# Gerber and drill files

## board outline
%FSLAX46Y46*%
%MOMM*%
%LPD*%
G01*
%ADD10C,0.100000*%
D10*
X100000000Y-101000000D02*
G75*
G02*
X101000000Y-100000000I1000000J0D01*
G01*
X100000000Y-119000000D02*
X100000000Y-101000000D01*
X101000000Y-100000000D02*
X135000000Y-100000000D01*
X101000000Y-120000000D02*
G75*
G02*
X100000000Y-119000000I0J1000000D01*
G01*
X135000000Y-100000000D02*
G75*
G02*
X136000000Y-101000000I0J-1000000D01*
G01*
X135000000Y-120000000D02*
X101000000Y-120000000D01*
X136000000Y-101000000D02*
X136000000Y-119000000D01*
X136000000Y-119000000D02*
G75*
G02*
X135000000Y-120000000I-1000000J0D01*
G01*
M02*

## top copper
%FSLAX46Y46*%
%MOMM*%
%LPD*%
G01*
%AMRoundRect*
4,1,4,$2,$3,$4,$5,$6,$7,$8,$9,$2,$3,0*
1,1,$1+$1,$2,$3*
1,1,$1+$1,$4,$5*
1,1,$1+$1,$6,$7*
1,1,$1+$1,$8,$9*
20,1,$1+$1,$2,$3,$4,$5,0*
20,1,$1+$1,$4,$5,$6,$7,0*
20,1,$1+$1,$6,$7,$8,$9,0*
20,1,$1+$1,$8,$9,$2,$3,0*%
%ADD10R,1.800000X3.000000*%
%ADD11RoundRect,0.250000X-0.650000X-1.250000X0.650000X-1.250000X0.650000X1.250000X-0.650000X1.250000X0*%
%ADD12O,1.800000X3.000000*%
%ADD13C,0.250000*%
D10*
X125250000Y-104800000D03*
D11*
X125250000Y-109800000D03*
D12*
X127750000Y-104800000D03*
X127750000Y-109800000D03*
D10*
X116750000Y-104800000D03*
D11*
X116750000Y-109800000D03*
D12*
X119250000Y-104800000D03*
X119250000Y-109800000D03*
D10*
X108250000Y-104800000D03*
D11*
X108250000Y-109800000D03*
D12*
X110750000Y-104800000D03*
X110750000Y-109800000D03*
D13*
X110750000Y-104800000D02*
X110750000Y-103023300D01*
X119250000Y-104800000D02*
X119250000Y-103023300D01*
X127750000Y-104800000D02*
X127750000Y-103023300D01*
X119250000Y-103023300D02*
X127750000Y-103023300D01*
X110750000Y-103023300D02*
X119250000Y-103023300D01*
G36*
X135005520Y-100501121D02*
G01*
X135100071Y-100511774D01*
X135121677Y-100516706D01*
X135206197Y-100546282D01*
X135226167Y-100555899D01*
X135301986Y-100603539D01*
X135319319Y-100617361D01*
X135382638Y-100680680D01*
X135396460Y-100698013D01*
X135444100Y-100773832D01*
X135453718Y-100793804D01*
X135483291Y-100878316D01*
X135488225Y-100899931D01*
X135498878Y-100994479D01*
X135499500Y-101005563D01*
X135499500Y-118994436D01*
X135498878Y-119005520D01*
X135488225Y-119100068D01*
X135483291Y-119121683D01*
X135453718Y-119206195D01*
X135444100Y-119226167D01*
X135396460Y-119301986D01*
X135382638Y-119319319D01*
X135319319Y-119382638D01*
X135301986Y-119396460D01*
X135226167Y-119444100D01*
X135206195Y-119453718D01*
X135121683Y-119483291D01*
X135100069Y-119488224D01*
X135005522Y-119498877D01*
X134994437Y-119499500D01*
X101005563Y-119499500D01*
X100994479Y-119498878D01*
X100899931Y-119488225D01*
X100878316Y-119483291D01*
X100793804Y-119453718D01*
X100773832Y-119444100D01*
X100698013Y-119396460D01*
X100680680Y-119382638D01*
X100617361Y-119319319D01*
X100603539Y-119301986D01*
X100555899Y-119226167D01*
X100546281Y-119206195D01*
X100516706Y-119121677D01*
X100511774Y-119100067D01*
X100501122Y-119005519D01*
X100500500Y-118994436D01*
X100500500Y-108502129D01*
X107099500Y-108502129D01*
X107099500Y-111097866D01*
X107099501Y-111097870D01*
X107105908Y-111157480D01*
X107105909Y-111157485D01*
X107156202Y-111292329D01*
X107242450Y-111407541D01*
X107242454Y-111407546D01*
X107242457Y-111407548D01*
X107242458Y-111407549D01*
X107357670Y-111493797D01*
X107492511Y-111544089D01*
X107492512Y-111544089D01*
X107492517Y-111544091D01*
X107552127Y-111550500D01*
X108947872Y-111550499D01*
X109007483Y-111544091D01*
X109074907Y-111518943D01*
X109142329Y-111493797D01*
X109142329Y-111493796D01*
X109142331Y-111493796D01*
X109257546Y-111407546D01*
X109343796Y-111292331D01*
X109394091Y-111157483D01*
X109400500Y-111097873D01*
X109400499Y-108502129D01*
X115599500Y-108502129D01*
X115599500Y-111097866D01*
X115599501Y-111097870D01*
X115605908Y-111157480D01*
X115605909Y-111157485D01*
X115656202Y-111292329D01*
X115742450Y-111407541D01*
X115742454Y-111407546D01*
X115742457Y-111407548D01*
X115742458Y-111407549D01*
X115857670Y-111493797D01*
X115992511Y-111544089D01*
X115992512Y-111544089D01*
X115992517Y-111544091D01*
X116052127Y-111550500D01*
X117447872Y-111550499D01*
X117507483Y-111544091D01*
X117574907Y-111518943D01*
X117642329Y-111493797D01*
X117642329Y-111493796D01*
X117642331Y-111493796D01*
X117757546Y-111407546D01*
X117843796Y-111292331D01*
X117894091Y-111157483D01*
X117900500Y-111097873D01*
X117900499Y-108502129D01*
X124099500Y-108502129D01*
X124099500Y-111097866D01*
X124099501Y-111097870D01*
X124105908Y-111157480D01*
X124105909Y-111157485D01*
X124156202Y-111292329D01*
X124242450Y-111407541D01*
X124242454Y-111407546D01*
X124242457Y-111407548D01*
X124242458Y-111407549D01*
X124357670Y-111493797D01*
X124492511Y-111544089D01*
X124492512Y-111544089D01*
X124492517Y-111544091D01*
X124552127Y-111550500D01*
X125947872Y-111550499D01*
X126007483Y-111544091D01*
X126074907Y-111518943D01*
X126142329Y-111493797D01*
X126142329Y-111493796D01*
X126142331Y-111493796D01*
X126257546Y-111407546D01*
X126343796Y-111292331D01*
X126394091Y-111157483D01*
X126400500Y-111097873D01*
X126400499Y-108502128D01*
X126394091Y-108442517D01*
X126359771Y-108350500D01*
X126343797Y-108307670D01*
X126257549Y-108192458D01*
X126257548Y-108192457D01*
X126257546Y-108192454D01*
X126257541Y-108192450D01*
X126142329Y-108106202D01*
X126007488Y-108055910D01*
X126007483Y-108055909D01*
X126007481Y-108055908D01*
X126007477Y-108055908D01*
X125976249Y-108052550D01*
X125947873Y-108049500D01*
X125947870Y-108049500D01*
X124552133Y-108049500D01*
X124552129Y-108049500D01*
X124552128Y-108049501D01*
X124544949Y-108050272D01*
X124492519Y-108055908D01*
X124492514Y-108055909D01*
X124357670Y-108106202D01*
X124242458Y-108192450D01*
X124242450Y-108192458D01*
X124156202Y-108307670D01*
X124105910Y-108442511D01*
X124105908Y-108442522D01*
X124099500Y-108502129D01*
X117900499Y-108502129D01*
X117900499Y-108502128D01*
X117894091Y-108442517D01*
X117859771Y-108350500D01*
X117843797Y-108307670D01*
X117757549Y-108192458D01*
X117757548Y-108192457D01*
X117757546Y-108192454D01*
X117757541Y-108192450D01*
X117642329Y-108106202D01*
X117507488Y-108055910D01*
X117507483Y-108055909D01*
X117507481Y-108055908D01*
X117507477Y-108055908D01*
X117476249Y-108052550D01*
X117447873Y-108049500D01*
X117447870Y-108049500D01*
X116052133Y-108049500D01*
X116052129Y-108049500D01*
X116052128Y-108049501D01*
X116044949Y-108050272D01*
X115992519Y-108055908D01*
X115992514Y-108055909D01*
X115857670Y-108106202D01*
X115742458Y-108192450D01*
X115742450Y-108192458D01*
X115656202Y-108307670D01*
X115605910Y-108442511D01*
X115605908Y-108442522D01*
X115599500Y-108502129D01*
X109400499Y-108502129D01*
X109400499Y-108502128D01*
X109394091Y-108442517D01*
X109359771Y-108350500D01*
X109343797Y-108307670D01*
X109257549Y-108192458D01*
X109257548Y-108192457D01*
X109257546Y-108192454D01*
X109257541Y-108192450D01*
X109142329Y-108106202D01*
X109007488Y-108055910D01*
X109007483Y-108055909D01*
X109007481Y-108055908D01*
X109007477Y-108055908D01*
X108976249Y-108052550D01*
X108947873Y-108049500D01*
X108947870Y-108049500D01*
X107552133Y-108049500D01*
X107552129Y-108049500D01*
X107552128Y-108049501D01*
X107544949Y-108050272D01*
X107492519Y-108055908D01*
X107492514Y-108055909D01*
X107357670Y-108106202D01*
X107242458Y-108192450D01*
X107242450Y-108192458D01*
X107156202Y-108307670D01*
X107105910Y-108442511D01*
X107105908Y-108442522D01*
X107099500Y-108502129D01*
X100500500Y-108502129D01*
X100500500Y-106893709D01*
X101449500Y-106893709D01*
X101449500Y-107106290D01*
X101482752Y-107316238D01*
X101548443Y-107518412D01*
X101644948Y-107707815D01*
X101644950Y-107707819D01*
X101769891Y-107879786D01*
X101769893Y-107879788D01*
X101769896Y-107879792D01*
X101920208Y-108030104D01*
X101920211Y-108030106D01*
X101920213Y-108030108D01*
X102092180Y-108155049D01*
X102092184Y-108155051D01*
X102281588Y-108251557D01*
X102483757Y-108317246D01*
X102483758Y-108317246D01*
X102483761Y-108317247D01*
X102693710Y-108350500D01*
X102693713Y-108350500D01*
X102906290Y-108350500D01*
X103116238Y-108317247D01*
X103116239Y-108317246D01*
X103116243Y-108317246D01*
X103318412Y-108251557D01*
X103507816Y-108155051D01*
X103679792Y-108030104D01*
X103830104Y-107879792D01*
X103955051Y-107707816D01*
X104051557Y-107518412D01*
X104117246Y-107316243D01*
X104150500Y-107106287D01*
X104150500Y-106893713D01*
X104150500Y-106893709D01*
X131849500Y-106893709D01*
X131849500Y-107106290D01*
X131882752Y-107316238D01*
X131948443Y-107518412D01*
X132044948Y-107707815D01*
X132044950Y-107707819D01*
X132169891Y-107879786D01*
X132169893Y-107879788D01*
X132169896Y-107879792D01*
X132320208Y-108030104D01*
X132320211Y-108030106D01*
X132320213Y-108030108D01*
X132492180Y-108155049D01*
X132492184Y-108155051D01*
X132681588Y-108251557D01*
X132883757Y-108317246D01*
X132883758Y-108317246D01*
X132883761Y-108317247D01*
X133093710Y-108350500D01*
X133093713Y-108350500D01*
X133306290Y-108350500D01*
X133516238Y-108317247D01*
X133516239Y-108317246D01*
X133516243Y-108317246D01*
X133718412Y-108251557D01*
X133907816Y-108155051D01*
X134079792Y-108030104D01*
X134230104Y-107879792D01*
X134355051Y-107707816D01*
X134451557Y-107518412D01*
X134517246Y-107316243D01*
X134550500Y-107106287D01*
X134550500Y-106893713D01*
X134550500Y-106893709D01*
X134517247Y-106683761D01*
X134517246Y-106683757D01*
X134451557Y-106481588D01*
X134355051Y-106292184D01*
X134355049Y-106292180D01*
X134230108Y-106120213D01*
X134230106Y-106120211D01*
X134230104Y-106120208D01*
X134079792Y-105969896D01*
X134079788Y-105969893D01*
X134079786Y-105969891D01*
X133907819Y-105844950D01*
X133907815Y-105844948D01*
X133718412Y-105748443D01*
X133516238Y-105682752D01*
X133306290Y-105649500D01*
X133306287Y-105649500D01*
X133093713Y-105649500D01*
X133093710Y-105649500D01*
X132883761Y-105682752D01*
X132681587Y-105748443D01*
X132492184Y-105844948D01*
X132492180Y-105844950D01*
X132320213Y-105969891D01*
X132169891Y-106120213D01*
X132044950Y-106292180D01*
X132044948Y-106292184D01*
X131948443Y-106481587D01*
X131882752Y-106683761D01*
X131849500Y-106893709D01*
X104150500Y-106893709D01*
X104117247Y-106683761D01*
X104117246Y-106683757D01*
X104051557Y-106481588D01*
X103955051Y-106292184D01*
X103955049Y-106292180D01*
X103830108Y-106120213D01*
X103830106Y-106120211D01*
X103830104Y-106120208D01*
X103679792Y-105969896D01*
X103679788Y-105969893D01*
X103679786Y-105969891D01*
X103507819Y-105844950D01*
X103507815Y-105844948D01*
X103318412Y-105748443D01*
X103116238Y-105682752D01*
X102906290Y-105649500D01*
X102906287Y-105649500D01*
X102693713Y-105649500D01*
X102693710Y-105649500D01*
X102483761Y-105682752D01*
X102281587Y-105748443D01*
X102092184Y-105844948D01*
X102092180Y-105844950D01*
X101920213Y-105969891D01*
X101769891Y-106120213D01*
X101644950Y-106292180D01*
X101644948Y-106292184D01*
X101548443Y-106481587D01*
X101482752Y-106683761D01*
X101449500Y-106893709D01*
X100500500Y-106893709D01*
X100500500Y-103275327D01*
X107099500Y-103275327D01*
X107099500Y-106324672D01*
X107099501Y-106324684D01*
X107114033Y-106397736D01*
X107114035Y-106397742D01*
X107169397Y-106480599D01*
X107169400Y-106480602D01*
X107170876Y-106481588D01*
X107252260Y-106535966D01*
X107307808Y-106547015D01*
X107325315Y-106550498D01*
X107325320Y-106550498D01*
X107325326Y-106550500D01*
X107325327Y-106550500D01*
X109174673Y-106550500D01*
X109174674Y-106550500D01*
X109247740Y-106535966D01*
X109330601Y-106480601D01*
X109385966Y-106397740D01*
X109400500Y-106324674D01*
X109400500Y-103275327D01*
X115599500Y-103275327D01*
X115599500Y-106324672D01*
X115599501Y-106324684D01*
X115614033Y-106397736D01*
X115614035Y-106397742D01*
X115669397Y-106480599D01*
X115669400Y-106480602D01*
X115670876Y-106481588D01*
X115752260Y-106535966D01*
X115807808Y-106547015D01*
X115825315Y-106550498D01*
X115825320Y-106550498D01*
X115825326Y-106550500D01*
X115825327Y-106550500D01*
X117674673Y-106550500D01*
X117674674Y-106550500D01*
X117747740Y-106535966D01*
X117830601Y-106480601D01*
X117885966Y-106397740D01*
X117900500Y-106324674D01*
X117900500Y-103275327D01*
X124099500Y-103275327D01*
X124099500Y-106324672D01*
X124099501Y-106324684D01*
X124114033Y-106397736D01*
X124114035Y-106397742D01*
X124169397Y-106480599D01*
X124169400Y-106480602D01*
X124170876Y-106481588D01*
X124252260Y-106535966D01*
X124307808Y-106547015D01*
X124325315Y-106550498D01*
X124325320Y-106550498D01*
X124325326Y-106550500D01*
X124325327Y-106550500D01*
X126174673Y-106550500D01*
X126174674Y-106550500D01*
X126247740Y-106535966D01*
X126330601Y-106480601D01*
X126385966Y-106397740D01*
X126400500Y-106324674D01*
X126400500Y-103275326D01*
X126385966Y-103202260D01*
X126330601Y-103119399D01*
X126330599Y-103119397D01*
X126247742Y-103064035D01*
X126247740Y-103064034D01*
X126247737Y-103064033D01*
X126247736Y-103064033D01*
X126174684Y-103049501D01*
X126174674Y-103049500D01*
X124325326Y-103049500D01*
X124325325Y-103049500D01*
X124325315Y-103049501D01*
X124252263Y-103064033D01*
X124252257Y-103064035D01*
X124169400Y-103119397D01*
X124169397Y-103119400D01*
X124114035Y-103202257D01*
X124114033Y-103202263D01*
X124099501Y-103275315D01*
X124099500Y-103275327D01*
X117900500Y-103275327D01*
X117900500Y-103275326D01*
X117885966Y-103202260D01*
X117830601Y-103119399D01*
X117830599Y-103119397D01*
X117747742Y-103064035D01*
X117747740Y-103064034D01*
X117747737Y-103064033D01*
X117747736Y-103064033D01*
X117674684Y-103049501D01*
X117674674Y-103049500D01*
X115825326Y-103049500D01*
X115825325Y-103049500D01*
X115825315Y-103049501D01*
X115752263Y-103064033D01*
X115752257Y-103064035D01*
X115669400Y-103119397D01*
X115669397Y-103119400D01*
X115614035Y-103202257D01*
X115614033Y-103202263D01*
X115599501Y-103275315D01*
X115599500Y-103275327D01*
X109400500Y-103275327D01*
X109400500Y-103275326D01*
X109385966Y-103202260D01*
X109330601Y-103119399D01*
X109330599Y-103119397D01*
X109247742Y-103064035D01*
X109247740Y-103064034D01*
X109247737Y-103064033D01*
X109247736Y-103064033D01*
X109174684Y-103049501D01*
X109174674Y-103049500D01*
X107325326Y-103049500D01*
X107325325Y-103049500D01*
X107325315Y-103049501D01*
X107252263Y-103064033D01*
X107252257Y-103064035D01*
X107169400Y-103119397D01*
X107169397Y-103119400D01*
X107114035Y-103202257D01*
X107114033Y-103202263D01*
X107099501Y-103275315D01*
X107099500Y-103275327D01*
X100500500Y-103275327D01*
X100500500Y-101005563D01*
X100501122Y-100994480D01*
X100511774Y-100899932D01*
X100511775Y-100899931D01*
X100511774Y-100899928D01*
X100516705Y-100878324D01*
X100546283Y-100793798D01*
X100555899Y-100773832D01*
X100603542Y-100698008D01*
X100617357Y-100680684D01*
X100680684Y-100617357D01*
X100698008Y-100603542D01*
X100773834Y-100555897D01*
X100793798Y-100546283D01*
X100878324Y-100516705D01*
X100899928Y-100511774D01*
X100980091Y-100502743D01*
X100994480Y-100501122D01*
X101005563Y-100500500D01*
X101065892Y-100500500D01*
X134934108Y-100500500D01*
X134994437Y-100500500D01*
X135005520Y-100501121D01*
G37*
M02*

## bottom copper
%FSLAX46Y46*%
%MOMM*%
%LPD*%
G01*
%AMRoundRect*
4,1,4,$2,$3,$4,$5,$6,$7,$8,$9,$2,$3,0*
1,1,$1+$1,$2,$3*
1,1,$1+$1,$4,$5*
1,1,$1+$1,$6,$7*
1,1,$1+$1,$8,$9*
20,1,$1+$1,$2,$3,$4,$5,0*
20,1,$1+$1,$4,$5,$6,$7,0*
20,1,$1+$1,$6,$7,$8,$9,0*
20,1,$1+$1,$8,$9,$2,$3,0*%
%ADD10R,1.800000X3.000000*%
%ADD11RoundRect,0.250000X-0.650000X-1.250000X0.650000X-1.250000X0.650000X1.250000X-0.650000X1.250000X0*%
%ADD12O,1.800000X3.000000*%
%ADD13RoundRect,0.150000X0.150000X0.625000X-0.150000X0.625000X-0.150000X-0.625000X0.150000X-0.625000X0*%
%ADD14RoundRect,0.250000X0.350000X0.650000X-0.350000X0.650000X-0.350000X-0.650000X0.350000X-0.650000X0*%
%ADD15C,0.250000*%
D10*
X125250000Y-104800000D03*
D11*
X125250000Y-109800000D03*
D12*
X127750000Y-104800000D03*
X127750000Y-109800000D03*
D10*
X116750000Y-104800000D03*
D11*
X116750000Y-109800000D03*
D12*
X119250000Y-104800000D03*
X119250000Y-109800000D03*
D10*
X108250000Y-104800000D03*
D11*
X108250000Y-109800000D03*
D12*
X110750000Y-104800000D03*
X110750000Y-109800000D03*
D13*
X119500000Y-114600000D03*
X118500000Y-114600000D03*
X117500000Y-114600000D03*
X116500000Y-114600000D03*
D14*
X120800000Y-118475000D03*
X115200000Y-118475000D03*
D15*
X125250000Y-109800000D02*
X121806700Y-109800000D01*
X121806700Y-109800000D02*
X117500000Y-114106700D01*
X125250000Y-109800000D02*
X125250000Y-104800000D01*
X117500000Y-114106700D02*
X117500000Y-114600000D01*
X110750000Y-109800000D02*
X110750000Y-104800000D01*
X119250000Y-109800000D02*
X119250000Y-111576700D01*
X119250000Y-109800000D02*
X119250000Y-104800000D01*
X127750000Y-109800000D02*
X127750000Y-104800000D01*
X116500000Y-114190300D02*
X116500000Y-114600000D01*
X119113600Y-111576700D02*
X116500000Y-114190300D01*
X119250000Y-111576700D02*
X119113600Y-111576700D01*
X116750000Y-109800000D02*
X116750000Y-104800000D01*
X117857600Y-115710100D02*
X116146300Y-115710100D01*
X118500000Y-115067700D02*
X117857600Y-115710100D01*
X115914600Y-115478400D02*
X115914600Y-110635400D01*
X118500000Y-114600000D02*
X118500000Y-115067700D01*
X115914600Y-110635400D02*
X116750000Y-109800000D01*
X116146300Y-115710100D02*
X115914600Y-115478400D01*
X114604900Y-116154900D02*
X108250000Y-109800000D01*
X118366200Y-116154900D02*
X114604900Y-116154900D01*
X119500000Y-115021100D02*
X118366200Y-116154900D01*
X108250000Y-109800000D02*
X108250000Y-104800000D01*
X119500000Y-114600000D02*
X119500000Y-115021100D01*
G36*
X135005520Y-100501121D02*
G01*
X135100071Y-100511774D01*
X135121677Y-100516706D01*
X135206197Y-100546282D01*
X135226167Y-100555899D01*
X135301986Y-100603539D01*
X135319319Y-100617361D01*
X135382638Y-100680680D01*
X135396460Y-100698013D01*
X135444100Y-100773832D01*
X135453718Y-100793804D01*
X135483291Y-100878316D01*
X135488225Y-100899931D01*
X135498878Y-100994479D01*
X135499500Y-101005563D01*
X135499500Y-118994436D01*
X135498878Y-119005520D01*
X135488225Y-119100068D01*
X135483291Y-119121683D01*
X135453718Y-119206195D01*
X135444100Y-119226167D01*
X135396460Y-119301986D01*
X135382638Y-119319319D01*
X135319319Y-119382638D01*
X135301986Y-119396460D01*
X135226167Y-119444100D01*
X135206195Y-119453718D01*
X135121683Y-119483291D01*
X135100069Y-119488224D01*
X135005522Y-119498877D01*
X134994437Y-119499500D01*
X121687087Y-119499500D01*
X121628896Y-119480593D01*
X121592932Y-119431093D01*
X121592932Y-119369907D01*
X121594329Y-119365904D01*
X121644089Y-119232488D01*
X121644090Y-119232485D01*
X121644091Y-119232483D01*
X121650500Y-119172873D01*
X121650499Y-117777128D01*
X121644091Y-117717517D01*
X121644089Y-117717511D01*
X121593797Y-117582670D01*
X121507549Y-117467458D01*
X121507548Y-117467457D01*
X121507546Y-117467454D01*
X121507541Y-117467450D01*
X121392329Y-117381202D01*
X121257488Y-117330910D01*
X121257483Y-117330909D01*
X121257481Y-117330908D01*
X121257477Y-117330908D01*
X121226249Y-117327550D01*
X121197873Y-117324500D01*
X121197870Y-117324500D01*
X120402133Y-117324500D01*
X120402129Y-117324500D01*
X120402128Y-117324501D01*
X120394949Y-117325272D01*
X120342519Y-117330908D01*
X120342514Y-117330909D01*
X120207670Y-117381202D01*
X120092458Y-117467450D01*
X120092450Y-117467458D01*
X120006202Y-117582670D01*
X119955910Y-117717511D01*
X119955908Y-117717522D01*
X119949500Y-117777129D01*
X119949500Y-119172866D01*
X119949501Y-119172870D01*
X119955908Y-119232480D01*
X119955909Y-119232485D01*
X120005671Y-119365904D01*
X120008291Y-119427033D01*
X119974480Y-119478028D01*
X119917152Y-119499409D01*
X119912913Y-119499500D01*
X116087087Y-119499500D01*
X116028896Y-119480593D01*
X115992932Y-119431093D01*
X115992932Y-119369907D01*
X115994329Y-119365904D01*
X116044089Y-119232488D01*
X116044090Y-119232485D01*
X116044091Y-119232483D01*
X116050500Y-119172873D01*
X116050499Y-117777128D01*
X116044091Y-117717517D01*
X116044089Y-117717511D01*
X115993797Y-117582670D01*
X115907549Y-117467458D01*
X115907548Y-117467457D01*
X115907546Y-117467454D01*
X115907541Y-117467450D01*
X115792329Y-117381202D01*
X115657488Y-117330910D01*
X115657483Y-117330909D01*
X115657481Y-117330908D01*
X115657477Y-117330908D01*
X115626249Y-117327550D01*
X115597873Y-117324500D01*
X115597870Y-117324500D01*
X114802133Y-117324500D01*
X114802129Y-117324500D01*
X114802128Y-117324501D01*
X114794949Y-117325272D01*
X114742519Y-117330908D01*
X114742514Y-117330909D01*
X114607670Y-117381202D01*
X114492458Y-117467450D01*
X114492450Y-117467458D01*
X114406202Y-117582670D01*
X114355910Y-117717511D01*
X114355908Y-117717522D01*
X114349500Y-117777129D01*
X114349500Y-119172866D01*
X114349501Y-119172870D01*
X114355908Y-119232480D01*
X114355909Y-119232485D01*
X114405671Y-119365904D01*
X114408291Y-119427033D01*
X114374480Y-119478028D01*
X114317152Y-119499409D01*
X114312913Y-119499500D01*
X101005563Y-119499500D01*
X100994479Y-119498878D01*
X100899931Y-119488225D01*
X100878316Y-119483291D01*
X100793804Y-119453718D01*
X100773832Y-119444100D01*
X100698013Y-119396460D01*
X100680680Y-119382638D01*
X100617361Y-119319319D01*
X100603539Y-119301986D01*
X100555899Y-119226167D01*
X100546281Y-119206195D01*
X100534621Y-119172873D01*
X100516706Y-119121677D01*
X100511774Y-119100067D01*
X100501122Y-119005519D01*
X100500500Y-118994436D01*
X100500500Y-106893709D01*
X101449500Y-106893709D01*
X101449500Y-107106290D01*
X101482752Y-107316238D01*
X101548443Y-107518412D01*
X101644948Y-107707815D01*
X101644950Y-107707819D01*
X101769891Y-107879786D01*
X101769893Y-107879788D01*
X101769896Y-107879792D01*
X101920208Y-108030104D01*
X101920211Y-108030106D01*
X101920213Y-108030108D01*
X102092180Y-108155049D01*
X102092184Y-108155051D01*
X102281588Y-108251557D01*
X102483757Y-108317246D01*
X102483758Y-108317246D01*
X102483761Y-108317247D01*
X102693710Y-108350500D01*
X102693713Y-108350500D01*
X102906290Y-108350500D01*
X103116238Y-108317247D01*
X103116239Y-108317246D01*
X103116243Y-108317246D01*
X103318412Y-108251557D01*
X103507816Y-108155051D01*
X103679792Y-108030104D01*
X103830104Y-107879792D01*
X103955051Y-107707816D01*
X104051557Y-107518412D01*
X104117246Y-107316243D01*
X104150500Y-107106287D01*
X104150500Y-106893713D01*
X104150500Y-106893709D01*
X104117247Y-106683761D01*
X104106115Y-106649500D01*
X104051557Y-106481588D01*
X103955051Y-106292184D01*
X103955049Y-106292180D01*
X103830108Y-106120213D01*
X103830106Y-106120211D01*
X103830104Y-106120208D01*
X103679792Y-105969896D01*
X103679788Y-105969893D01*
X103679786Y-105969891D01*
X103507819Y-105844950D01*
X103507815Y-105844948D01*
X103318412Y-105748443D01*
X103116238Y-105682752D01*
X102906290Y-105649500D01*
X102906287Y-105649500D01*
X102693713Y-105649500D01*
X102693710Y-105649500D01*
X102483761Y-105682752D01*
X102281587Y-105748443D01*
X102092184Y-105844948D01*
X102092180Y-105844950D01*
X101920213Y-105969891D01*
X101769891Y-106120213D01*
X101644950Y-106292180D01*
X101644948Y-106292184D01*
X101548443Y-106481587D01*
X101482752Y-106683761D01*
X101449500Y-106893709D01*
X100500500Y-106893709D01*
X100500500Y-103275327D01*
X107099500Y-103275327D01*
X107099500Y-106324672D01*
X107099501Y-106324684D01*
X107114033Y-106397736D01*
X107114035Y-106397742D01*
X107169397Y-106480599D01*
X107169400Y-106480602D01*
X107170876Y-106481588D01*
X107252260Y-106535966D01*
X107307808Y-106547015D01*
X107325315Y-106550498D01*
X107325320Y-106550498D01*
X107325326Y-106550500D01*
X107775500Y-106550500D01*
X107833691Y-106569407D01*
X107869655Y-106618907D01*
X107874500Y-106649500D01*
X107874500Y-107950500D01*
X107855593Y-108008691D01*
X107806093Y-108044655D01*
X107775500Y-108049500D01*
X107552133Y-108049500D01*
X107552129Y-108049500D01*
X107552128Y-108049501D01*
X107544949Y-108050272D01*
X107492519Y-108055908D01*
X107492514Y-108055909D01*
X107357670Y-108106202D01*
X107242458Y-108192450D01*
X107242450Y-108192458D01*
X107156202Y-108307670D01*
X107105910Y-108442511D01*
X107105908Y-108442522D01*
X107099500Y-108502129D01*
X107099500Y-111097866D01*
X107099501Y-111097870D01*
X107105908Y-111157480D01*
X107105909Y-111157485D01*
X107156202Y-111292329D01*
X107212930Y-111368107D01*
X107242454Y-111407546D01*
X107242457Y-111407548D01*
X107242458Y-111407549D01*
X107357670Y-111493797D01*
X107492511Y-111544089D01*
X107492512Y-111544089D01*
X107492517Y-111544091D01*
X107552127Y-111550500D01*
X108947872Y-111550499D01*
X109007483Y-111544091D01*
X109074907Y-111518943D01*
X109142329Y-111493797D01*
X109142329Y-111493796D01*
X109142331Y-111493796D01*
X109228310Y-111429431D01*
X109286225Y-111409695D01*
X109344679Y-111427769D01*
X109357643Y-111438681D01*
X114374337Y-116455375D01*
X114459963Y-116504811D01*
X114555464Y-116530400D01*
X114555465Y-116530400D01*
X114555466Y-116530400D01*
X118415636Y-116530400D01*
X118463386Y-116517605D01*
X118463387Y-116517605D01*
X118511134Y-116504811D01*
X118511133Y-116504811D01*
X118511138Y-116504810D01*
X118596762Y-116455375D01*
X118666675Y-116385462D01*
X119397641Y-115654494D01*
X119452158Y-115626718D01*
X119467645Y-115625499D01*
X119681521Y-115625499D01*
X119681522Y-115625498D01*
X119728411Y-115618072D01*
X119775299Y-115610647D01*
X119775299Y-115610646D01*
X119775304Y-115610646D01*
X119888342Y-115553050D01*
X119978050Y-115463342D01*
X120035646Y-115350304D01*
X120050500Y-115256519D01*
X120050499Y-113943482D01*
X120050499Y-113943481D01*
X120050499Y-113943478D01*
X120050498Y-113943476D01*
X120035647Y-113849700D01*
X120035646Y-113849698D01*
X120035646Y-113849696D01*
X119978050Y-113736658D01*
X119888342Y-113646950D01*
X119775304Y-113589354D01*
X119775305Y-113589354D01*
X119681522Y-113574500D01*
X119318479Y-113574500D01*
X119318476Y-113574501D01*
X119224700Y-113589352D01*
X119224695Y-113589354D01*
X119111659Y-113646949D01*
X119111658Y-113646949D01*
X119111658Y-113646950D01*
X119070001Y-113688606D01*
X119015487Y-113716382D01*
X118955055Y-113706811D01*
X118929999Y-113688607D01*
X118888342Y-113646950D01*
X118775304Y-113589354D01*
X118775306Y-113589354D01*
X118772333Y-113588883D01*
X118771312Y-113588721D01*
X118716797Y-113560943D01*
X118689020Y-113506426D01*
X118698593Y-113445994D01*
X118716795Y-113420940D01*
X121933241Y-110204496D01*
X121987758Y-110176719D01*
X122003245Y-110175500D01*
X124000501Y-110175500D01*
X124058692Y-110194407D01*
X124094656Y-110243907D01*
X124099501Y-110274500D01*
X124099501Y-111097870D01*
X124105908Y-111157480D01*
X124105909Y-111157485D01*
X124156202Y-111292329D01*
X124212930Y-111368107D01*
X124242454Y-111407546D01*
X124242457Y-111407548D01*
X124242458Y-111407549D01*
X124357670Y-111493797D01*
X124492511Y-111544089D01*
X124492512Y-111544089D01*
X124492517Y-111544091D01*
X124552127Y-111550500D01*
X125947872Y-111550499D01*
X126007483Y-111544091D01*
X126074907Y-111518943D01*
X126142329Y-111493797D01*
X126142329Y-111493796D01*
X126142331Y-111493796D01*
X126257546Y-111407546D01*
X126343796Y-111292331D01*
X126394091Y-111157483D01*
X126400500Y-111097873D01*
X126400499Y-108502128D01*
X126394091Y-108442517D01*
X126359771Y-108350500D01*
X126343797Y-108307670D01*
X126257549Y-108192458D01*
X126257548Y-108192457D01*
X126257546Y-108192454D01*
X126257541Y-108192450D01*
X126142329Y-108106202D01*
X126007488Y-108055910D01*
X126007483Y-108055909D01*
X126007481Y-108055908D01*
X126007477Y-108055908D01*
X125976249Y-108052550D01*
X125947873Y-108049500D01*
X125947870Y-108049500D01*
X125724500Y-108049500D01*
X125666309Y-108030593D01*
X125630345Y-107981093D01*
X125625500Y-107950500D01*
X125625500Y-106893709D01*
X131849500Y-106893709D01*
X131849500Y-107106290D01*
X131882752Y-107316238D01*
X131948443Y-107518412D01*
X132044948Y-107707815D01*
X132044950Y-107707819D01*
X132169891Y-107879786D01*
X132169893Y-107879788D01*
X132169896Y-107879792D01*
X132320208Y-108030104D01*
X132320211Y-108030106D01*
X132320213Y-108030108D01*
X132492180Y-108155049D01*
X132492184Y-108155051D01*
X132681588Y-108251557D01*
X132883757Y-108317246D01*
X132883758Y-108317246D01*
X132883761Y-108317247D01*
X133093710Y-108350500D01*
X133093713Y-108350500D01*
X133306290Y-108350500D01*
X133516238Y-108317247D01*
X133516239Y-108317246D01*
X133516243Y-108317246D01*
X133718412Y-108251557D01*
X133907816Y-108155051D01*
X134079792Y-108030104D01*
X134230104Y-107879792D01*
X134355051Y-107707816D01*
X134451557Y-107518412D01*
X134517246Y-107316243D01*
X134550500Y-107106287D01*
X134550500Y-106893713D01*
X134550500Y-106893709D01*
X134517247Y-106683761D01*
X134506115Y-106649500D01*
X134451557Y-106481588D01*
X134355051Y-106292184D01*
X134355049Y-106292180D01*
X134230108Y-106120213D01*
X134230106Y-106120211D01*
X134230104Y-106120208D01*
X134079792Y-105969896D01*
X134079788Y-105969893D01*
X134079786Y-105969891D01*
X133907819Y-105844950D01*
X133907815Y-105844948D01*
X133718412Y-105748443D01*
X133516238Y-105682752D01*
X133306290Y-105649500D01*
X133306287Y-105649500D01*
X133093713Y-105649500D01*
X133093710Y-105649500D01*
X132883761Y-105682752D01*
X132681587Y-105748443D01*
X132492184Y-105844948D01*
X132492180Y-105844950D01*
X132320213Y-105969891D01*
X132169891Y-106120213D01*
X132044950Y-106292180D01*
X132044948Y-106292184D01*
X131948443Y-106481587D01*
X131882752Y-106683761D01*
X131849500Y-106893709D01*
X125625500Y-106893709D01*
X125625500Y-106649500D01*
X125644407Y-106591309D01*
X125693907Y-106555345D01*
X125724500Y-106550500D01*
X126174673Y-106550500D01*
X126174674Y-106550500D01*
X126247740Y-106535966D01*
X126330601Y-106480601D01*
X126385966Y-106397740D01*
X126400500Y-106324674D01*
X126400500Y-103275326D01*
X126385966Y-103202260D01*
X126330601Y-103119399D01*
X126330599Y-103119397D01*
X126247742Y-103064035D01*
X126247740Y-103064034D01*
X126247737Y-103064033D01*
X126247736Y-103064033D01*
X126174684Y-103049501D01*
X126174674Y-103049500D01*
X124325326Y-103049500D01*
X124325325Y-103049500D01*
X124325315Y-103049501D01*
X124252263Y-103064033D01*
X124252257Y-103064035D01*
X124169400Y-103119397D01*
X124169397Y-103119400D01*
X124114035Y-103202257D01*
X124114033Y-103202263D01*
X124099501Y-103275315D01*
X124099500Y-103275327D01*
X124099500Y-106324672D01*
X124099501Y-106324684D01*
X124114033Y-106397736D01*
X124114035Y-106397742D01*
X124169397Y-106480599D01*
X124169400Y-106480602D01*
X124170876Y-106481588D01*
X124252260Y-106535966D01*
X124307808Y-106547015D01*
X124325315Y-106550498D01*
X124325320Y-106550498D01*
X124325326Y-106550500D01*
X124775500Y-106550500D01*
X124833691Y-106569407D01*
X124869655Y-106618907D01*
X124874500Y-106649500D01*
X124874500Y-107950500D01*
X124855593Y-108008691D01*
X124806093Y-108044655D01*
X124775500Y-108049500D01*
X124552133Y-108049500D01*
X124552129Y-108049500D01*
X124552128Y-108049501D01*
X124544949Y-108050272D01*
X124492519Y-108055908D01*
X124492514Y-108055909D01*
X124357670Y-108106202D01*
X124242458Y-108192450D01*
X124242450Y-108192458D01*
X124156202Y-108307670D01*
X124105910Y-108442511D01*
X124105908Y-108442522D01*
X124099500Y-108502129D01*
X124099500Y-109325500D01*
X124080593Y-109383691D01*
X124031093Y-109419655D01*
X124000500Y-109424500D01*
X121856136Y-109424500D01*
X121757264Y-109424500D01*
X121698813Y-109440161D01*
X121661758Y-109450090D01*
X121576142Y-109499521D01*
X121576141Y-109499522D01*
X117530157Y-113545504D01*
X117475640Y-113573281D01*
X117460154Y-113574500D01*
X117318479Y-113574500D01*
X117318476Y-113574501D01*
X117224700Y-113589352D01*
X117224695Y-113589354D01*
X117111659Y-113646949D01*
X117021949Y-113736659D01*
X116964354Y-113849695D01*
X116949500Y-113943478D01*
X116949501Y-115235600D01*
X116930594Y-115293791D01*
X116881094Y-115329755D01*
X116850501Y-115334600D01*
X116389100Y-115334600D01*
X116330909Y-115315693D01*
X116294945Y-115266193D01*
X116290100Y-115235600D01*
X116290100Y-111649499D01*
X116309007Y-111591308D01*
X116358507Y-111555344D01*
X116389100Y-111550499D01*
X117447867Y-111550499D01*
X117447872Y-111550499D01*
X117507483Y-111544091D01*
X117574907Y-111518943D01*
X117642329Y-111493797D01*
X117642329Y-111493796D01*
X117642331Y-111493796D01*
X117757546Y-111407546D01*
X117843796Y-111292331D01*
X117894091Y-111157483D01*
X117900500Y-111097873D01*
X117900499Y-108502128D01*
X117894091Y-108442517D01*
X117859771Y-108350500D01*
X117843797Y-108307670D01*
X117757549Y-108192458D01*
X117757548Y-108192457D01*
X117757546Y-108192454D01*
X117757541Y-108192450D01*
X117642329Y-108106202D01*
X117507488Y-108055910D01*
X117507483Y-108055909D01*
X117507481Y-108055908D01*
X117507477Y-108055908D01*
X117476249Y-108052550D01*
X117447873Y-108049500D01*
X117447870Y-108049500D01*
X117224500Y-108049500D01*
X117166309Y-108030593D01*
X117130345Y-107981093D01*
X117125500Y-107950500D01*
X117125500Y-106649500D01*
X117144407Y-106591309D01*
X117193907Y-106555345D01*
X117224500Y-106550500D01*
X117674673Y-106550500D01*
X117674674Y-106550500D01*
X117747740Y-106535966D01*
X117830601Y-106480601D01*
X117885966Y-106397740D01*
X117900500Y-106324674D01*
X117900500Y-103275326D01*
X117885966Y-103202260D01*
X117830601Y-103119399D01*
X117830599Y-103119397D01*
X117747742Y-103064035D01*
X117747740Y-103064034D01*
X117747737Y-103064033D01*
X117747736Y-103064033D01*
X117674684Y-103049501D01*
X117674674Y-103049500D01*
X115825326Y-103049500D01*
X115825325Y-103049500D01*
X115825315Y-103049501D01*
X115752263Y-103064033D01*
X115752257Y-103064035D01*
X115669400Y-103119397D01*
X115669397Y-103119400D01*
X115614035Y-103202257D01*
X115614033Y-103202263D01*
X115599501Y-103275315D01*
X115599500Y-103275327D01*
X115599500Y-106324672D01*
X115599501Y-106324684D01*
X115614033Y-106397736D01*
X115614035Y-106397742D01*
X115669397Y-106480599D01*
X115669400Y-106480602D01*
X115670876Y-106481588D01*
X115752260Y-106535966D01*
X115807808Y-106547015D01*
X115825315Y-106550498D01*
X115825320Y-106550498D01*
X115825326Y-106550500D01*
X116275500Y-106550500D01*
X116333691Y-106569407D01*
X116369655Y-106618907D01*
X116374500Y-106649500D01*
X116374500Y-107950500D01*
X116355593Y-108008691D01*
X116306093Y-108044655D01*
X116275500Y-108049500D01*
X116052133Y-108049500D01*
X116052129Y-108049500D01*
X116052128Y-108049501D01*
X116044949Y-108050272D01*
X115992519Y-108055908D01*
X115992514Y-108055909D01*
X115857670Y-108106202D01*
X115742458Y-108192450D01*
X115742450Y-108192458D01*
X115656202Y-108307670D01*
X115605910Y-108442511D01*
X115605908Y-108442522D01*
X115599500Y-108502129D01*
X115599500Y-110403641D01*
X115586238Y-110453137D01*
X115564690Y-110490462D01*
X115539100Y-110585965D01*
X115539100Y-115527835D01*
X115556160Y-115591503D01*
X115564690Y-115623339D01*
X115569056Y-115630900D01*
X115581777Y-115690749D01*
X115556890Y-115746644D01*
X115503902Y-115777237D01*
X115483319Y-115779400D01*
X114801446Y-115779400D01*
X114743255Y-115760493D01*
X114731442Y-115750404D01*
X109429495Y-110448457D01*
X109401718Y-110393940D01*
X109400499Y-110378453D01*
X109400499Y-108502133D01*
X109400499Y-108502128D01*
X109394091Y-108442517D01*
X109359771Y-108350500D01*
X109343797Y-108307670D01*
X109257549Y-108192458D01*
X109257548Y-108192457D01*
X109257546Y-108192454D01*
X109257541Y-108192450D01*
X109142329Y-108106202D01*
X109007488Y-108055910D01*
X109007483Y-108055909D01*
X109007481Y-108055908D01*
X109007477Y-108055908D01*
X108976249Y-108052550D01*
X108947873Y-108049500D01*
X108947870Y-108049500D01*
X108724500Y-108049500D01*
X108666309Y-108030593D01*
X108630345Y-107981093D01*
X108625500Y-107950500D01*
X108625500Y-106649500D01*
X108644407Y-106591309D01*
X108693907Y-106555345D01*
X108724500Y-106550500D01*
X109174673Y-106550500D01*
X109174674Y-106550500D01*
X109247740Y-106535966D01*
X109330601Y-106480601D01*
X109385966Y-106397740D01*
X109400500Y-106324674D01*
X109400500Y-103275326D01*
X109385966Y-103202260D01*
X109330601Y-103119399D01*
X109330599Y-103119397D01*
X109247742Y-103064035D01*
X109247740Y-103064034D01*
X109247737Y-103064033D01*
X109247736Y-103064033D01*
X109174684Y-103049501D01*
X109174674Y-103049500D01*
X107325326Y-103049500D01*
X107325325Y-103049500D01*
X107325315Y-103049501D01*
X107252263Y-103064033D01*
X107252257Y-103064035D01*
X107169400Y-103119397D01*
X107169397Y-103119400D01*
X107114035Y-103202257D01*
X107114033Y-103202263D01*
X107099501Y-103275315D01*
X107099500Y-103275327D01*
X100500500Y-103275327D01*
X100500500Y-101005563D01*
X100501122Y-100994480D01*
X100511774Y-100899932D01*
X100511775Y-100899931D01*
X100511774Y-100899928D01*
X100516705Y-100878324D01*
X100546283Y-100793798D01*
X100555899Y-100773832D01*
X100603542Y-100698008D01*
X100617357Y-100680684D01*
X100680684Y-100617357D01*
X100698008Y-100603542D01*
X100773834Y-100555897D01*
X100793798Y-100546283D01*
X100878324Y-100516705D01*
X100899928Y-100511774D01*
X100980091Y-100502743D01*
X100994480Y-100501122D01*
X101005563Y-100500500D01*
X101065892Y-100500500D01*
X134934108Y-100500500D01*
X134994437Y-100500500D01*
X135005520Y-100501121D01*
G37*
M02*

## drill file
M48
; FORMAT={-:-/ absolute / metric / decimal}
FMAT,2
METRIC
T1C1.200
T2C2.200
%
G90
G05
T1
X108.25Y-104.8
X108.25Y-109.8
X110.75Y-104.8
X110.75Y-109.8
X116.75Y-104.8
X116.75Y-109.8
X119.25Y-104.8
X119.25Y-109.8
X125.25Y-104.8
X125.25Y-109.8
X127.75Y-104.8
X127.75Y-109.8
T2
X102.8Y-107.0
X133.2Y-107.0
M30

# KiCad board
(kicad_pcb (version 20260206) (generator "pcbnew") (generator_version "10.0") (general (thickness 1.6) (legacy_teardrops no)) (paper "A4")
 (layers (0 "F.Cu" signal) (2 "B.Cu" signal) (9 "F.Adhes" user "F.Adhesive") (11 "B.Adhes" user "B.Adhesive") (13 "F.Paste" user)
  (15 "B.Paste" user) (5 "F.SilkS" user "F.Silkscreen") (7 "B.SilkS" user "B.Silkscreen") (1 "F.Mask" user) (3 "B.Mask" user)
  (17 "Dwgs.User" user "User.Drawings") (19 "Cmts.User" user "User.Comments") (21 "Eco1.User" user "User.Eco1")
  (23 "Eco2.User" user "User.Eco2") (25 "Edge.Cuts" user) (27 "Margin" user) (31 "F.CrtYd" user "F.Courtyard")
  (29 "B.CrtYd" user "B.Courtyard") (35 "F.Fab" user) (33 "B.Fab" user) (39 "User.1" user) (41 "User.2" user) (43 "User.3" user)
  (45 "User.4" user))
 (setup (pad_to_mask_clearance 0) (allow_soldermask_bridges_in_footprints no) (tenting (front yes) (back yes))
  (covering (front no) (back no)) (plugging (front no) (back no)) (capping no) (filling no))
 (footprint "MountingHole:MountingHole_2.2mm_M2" (layer "F.Cu") (at 102.8 107)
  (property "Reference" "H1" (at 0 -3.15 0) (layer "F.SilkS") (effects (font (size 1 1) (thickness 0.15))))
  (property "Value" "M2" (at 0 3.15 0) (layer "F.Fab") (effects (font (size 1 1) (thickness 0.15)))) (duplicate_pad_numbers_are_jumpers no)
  (pad "" np_thru_hole circle (at 0 0) (size 2.2 2.2) (drill 2.2) (layers "*.Cu" "*.Mask") (zone_connect 2)))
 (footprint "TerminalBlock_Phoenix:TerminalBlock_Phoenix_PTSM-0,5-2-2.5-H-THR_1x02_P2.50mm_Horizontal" (layer "F.Cu") (at 125.25 109.8)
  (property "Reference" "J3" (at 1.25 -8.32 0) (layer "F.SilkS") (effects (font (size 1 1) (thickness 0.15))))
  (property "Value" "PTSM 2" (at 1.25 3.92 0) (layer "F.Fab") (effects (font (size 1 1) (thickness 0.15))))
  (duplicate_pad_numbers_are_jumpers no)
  (pad "1" thru_hole rect (at 0 -5) (size 1.8 3) (drill 1.2) (layers "*.Cu" "*.Mask") (remove_unused_layers no) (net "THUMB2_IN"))
  (pad "1" thru_hole roundrect (at 0 0) (size 1.8 3) (drill 1.2) (layers "*.Cu" "*.Mask") (remove_unused_layers no)
   (roundrect_rratio 0.138889) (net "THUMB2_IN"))
  (pad "2" thru_hole oval (at 2.5 -5) (size 1.8 3) (drill 1.2) (layers "*.Cu" "*.Mask") (remove_unused_layers no) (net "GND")
   (zone_connect 2))
  (pad "2" thru_hole oval (at 2.5 0) (size 1.8 3) (drill 1.2) (layers "*.Cu" "*.Mask") (remove_unused_layers no) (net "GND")
   (zone_connect 2)))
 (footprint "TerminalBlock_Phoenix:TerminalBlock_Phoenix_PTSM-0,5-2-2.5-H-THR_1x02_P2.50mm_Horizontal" (layer "F.Cu") (at 116.75 109.8)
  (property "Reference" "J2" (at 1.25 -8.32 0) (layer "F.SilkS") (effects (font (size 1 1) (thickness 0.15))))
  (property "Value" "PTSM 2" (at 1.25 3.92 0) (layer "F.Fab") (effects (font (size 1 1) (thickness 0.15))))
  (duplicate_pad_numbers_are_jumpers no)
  (pad "1" thru_hole rect (at 0 -5) (size 1.8 3) (drill 1.2) (layers "*.Cu" "*.Mask") (remove_unused_layers no) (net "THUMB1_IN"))
  (pad "1" thru_hole roundrect (at 0 0) (size 1.8 3) (drill 1.2) (layers "*.Cu" "*.Mask") (remove_unused_layers no)
   (roundrect_rratio 0.138889) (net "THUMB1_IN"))
  (pad "2" thru_hole oval (at 2.5 -5) (size 1.8 3) (drill 1.2) (layers "*.Cu" "*.Mask") (remove_unused_layers no) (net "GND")
   (zone_connect 2))
  (pad "2" thru_hole oval (at 2.5 0) (size 1.8 3) (drill 1.2) (layers "*.Cu" "*.Mask") (remove_unused_layers no) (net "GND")
   (zone_connect 2)))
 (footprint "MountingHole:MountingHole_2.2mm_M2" (layer "F.Cu") (at 133.2 107)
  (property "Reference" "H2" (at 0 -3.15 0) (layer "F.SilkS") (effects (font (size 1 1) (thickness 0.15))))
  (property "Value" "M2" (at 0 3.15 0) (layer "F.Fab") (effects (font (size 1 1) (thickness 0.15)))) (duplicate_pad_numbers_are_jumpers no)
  (pad "" np_thru_hole circle (at 0 0) (size 2.2 2.2) (drill 2.2) (layers "*.Cu" "*.Mask") (zone_connect 2)))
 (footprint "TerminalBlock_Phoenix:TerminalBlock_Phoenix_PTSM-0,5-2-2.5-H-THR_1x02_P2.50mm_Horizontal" (layer "F.Cu") (at 108.25 109.8)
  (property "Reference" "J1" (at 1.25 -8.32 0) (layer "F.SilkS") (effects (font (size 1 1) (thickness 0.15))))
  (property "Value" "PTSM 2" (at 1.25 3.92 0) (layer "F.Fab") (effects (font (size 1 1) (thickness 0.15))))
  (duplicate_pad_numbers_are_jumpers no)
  (pad "1" thru_hole rect (at 0 -5) (size 1.8 3) (drill 1.2) (layers "*.Cu" "*.Mask") (remove_unused_layers no) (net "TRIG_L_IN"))
  (pad "1" thru_hole roundrect (at 0 0) (size 1.8 3) (drill 1.2) (layers "*.Cu" "*.Mask") (remove_unused_layers no)
   (roundrect_rratio 0.138889) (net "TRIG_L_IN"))
  (pad "2" thru_hole oval (at 2.5 -5) (size 1.8 3) (drill 1.2) (layers "*.Cu" "*.Mask") (remove_unused_layers no) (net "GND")
   (zone_connect 2))
  (pad "2" thru_hole oval (at 2.5 0) (size 1.8 3) (drill 1.2) (layers "*.Cu" "*.Mask") (remove_unused_layers no) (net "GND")
   (zone_connect 2)))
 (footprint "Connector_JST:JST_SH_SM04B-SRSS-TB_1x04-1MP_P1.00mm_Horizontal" (layer "B.Cu") (at 118 116.6 180)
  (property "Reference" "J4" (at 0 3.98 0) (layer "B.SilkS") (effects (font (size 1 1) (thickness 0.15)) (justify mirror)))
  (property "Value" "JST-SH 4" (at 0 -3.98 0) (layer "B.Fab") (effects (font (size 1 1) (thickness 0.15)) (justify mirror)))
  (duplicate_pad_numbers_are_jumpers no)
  (pad "1" smd roundrect (at -1.5 2 180) (size 0.6 1.55) (layers "B.Cu" "B.Mask" "B.Paste") (roundrect_rratio 0.25) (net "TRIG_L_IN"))
  (pad "2" smd roundrect (at -0.5 2 180) (size 0.6 1.55) (layers "B.Cu" "B.Mask" "B.Paste") (roundrect_rratio 0.25) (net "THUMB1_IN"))
  (pad "3" smd roundrect (at 0.5 2 180) (size 0.6 1.55) (layers "B.Cu" "B.Mask" "B.Paste") (roundrect_rratio 0.25) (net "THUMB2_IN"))
  (pad "4" smd roundrect (at 1.5 2 180) (size 0.6 1.55) (layers "B.Cu" "B.Mask" "B.Paste") (roundrect_rratio 0.25) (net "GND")
   (zone_connect 2))
  (pad "MP" smd roundrect (at -2.8 -1.875 180) (size 1.2 1.8) (layers "B.Cu" "B.Mask" "B.Paste") (roundrect_rratio 0.208333)
   (zone_connect 2))
  (pad "MP" smd roundrect (at 2.8 -1.875 180) (size 1.2 1.8) (layers "B.Cu" "B.Mask" "B.Paste") (roundrect_rratio 0.208333) (zone_connect 2)))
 (gr_arc (start 100 101) (mid 100.292893 100.292893) (end 101 100) (stroke (width 0.1) (type default)) (layer "Edge.Cuts"))
 (gr_line (start 100 119) (end 100 101) (stroke (width 0.1) (type default)) (layer "Edge.Cuts"))
 (gr_line (start 101 100) (end 135 100) (stroke (width 0.1) (type default)) (layer "Edge.Cuts"))
 (gr_arc (start 101 120) (mid 100.292893 119.707107) (end 100 119) (stroke (width 0.1) (type default)) (layer "Edge.Cuts"))
 (gr_arc (start 135 100) (mid 135.707107 100.292893) (end 136 101) (stroke (width 0.1) (type default)) (layer "Edge.Cuts"))
 (gr_line (start 135 120) (end 101 120) (stroke (width 0.1) (type default)) (layer "Edge.Cuts"))
 (gr_line (start 136 101) (end 136 119) (stroke (width 0.1) (type default)) (layer "Edge.Cuts"))
 (gr_arc (start 136 119) (mid 135.707107 119.707107) (end 135 120) (stroke (width 0.1) (type default)) (layer "Edge.Cuts"))
 (segment (start 125.25 109.8) (end 121.8067 109.8) (width 0.25) (layer "B.Cu") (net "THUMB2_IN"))
 (segment (start 121.8067 109.8) (end 117.5 114.1067) (width 0.25) (layer "B.Cu") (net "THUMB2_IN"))
 (segment (start 125.25 109.8) (end 125.25 104.8) (width 0.25) (layer "B.Cu") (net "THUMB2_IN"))
 (segment (start 117.5 114.1067) (end 117.5 114.6) (width 0.25) (layer "B.Cu") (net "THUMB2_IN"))
 (segment (start 110.75 104.8) (end 110.75 103.0233) (width 0.25) (layer "F.Cu") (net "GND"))
 (segment (start 119.25 104.8) (end 119.25 103.0233) (width 0.25) (layer "F.Cu") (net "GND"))
 (segment (start 127.75 104.8) (end 127.75 103.0233) (width 0.25) (layer "F.Cu") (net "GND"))
 (segment (start 119.25 103.0233) (end 127.75 103.0233) (width 0.25) (layer "F.Cu") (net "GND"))
 (segment (start 110.75 103.0233) (end 119.25 103.0233) (width 0.25) (layer "F.Cu") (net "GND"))
 (segment (start 110.75 109.8) (end 110.75 104.8) (width 0.25) (layer "B.Cu") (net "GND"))
 (segment (start 119.25 109.8) (end 119.25 111.5767) (width 0.25) (layer "B.Cu") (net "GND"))
 (segment (start 119.25 109.8) (end 119.25 104.8) (width 0.25) (layer "B.Cu") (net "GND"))
 (segment (start 127.75 109.8) (end 127.75 104.8) (width 0.25) (layer "B.Cu") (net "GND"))
 (segment (start 116.5 114.1903) (end 116.5 114.6) (width 0.25) (layer "B.Cu") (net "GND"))
 (segment (start 119.1136 111.5767) (end 116.5 114.1903) (width 0.25) (layer "B.Cu") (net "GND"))
 (segment (start 119.25 111.5767) (end 119.1136 111.5767) (width 0.25) (layer "B.Cu") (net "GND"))
 (segment (start 116.75 109.8) (end 116.75 104.8) (width 0.25) (layer "B.Cu") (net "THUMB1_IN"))
 (segment (start 117.8576 115.7101) (end 116.1463 115.7101) (width 0.25) (layer "B.Cu") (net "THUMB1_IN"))
 (segment (start 118.5 115.0677) (end 117.8576 115.7101) (width 0.25) (layer "B.Cu") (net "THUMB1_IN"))
 (segment (start 115.9146 115.4784) (end 115.9146 110.6354) (width 0.25) (layer "B.Cu") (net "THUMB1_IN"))
 (segment (start 118.5 114.6) (end 118.5 115.0677) (width 0.25) (layer "B.Cu") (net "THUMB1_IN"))
 (segment (start 115.9146 110.6354) (end 116.75 109.8) (width 0.25) (layer "B.Cu") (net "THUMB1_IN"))
 (segment (start 116.1463 115.7101) (end 115.9146 115.4784) (width 0.25) (layer "B.Cu") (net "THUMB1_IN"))
 (segment (start 114.6049 116.1549) (end 108.25 109.8) (width 0.25) (layer "B.Cu") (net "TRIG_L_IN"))
 (segment (start 118.3662 116.1549) (end 114.6049 116.1549) (width 0.25) (layer "B.Cu") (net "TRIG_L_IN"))
 (segment (start 119.5 115.0211) (end 118.3662 116.1549) (width 0.25) (layer "B.Cu") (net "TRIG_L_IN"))
 (segment (start 108.25 109.8) (end 108.25 104.8) (width 0.25) (layer "B.Cu") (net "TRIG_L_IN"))
 (segment (start 119.5 114.6) (end 119.5 115.0211) (width 0.25) (layer "B.Cu") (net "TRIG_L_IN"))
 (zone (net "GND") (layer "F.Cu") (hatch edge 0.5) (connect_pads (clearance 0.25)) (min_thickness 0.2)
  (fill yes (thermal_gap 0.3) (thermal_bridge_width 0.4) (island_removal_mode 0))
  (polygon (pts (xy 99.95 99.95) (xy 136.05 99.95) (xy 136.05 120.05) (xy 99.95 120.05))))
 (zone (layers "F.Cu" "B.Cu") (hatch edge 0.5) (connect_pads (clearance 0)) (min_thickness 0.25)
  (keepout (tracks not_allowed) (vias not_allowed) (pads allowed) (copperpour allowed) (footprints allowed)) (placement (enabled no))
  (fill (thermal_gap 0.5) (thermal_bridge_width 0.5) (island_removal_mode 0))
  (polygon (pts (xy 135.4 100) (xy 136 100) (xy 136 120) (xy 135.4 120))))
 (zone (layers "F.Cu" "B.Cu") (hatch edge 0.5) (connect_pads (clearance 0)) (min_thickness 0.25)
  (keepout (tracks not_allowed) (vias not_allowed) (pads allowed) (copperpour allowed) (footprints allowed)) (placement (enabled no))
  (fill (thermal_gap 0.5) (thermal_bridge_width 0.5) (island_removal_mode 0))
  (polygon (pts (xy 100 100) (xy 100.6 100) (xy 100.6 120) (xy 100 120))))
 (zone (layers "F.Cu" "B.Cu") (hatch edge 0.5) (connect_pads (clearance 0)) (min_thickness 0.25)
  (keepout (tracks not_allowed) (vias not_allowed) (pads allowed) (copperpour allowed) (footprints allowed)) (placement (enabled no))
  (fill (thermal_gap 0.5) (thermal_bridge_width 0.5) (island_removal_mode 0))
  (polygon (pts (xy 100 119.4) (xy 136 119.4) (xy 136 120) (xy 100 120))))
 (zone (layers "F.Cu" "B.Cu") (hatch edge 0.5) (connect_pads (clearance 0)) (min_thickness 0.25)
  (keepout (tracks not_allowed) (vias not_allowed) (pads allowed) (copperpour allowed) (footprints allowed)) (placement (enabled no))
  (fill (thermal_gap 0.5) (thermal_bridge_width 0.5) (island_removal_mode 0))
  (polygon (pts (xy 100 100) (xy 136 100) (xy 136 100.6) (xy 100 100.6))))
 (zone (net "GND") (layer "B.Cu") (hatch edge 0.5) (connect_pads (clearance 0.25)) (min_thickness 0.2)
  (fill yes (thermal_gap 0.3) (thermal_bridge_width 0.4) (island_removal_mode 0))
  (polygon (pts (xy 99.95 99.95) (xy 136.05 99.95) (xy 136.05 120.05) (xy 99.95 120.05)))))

